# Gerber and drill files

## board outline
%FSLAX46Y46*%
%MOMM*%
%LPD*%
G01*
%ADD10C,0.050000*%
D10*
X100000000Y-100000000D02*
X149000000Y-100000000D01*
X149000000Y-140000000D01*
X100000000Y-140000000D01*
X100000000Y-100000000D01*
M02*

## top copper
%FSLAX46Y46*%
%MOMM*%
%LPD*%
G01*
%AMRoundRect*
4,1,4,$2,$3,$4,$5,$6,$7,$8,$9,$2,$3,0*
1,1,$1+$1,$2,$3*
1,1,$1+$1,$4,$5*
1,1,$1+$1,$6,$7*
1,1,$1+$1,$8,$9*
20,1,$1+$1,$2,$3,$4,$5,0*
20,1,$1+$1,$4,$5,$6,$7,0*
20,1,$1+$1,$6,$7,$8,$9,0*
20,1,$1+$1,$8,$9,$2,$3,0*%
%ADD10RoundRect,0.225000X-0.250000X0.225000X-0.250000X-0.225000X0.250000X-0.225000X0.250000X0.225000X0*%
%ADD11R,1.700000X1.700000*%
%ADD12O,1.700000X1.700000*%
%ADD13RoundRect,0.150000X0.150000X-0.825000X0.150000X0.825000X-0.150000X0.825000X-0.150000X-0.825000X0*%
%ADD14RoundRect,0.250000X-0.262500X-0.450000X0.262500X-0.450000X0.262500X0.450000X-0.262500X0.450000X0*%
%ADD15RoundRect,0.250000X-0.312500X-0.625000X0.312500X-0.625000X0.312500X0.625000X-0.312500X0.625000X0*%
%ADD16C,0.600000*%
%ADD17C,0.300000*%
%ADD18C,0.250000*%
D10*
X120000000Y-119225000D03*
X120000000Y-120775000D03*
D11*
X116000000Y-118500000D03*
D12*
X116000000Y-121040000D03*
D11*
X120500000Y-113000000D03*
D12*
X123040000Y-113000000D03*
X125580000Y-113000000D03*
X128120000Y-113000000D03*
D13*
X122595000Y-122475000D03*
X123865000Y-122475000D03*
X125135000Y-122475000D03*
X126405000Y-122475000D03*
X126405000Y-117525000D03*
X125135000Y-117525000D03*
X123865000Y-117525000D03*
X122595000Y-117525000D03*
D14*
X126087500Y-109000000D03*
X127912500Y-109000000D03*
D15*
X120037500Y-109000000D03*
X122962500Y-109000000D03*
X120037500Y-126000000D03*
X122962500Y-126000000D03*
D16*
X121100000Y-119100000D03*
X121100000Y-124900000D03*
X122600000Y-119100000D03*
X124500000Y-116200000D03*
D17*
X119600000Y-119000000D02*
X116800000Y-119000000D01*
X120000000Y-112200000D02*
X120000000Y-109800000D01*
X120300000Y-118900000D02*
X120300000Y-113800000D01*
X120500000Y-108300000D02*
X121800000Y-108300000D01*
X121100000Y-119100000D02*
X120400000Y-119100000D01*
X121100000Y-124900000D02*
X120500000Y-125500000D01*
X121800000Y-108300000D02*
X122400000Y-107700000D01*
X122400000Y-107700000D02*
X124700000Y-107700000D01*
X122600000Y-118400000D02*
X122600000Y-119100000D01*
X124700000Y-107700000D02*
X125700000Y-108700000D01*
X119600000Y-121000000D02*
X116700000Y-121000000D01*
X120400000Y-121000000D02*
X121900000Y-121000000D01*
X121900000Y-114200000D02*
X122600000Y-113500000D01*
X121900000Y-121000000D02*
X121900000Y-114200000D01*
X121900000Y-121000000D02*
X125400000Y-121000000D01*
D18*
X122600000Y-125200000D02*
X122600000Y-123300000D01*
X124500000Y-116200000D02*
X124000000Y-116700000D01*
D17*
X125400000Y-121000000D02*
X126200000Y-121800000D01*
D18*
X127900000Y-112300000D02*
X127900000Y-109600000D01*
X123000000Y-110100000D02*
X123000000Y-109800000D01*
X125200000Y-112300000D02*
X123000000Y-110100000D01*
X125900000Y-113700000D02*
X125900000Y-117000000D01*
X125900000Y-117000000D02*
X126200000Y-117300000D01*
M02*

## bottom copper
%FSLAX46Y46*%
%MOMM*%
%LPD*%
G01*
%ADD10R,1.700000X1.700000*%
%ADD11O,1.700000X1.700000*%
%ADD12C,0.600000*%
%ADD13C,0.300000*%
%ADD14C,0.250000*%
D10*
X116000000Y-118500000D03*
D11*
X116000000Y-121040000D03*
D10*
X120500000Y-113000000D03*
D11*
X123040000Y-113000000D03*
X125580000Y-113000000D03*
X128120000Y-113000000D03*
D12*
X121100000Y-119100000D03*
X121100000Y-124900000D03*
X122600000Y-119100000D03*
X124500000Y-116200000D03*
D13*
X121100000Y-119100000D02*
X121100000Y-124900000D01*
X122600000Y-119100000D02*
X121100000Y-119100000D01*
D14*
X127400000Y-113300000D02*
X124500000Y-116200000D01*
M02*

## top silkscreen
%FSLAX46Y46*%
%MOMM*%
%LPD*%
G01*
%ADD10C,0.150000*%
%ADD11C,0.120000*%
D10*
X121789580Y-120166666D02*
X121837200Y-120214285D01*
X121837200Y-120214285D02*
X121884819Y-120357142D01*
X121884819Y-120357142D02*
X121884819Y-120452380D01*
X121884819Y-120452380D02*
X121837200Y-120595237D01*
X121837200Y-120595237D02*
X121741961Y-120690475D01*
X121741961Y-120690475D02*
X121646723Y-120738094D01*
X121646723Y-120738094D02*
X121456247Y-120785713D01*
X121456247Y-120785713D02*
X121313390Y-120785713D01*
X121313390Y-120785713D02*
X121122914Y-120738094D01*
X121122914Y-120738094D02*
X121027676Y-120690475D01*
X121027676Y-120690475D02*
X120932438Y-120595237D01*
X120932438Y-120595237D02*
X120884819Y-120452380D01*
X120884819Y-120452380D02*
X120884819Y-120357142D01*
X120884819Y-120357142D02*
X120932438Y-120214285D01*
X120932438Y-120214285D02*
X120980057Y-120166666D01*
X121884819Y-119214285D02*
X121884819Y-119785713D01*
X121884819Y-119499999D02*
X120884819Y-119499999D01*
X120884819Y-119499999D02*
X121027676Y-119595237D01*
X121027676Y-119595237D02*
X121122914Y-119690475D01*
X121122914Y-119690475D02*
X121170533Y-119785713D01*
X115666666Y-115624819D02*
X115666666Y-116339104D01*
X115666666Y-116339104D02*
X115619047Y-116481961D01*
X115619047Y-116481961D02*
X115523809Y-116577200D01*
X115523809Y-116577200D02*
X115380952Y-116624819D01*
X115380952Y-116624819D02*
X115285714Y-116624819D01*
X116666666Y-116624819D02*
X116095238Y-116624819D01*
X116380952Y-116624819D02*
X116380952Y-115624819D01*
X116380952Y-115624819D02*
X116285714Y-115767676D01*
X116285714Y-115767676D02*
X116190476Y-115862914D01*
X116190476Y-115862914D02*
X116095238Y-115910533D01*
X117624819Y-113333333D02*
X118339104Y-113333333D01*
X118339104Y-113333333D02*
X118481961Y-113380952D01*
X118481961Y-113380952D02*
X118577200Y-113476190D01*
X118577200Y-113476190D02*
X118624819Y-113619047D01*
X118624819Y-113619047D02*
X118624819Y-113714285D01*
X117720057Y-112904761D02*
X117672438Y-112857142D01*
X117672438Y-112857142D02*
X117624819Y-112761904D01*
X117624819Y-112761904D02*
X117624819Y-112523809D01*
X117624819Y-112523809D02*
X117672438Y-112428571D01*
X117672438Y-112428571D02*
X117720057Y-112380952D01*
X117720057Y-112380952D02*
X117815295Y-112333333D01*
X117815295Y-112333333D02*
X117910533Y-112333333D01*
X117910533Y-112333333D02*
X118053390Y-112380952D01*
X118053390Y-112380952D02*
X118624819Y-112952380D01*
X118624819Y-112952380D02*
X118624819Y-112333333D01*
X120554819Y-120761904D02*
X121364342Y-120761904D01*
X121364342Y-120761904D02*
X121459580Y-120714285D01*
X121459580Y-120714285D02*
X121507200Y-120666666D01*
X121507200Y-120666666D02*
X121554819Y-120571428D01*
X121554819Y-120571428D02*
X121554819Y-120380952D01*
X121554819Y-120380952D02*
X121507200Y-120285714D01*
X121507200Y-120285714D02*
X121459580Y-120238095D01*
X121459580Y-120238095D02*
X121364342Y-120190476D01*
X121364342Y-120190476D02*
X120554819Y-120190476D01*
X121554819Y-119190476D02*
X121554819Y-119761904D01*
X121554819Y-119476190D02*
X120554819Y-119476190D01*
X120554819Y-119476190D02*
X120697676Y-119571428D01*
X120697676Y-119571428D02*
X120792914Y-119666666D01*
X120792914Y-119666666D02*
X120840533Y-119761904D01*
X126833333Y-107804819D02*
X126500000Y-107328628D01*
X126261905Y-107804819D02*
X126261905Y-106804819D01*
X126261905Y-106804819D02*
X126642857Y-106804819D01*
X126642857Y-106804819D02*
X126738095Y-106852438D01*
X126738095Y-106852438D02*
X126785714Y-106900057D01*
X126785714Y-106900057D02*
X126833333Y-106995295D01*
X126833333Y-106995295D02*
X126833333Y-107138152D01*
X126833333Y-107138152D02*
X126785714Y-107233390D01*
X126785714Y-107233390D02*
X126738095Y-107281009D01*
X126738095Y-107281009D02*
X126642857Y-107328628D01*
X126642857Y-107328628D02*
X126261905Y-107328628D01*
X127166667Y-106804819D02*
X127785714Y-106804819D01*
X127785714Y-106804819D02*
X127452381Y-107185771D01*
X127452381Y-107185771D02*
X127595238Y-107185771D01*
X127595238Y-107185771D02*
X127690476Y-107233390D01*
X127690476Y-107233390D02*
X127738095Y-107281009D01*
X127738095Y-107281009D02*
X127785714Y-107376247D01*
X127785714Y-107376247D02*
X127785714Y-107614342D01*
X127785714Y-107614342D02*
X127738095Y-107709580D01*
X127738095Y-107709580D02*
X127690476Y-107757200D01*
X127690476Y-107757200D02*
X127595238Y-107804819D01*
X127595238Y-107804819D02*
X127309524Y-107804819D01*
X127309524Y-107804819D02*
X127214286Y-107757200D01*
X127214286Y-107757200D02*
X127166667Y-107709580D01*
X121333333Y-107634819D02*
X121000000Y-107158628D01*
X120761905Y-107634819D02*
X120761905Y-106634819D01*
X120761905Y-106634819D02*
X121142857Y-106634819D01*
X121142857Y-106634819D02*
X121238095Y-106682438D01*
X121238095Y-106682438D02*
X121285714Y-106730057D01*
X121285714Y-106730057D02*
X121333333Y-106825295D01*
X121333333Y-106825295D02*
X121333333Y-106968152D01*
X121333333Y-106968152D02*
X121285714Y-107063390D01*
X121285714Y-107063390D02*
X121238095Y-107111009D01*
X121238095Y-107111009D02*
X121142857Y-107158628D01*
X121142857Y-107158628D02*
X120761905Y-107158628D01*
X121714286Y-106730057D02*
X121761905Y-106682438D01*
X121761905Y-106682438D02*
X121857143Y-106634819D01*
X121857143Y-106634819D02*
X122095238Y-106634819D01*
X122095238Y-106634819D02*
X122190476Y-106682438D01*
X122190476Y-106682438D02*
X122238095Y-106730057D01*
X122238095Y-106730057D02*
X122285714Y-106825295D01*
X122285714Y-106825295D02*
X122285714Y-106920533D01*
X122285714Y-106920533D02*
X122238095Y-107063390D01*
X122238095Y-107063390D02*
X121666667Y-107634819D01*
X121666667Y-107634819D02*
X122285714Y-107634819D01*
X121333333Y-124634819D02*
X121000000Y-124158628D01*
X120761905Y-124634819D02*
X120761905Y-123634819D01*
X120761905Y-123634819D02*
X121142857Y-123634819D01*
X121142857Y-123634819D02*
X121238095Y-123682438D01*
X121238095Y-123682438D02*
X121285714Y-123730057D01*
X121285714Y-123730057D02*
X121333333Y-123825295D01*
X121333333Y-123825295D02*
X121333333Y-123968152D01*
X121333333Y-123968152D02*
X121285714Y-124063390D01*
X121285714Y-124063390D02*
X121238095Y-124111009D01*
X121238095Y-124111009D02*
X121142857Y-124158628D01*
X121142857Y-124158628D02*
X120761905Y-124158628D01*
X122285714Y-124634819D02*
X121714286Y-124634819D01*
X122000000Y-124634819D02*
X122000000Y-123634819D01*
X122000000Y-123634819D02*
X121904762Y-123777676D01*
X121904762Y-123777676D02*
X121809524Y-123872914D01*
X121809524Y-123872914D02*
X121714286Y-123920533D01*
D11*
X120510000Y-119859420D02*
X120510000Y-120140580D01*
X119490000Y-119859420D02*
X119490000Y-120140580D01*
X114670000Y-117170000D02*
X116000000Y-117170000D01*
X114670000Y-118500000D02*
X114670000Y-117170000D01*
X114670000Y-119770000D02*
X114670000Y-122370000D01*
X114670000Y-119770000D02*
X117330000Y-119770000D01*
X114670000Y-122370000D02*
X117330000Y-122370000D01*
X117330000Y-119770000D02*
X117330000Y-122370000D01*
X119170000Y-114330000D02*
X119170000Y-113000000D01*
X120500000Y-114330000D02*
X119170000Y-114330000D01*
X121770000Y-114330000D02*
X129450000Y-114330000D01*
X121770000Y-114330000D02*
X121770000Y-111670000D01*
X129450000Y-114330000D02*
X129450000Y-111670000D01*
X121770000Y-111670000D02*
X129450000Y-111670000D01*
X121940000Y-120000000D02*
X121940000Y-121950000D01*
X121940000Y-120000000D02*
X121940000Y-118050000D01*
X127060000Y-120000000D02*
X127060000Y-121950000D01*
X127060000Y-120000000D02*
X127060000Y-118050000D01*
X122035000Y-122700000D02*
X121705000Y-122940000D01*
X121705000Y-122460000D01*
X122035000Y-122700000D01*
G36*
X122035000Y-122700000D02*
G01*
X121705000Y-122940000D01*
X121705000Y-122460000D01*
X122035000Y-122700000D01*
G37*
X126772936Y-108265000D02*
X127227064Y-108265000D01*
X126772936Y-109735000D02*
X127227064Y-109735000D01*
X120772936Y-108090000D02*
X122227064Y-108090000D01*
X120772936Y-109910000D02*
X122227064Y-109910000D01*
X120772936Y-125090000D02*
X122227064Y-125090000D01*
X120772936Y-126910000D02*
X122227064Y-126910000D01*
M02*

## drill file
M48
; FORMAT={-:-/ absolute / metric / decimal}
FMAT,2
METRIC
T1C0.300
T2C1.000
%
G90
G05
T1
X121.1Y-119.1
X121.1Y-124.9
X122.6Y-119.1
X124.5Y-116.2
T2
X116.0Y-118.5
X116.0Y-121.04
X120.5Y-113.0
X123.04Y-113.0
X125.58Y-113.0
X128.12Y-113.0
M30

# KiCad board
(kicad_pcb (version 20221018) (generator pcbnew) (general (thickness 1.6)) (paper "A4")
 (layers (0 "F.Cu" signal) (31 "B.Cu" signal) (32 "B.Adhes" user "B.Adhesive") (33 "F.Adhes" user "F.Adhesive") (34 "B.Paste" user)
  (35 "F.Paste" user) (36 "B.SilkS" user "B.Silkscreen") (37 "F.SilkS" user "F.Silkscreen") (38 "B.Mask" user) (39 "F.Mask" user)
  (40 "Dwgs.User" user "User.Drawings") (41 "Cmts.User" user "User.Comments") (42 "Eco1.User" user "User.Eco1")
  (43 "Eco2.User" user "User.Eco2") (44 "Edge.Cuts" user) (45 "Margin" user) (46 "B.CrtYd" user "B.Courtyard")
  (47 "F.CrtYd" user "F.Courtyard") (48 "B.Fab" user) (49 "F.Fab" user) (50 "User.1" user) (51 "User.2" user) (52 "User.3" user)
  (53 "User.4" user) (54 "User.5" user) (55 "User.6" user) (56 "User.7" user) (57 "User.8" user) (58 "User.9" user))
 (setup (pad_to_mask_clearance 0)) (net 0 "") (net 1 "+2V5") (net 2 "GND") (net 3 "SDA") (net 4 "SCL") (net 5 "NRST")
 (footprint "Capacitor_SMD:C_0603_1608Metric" (layer "F.Cu") (at 120 120 -90)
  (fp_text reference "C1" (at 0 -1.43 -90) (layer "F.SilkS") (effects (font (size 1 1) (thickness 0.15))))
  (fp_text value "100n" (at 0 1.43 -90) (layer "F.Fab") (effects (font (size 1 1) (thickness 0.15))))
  (fp_line (start -0.14058 -0.51) (end 0.14058 -0.51) (stroke (width 0.12) (type solid)) (layer "F.SilkS"))
  (fp_line (start -0.14058 0.51) (end 0.14058 0.51) (stroke (width 0.12) (type solid)) (layer "F.SilkS"))
  (pad "1" smd roundrect (at -0.775 0 270) (size 0.9 0.95) (layers "F.Cu" "F.Paste" "F.Mask") (roundrect_rratio 0.25) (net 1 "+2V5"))
  (pad "2" smd roundrect (at 0.775 0 270) (size 0.9 0.95) (layers "F.Cu" "F.Paste" "F.Mask") (roundrect_rratio 0.25) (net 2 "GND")))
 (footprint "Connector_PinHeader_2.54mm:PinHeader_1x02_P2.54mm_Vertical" (layer "F.Cu") (at 116 118.5)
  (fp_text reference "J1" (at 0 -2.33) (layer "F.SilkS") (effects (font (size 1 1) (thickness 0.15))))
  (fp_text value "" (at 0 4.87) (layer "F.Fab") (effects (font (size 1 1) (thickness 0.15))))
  (fp_line (start -1.33 -1.33) (end 0 -1.33) (stroke (width 0.12) (type solid)) (layer "F.SilkS"))
  (fp_line (start -1.33 0) (end -1.33 -1.33) (stroke (width 0.12) (type solid)) (layer "F.SilkS"))
  (fp_line (start -1.33 1.27) (end -1.33 3.87) (stroke (width 0.12) (type solid)) (layer "F.SilkS"))
  (fp_line (start -1.33 1.27) (end 1.33 1.27) (stroke (width 0.12) (type solid)) (layer "F.SilkS"))
  (fp_line (start -1.33 3.87) (end 1.33 3.87) (stroke (width 0.12) (type solid)) (layer "F.SilkS"))
  (fp_line (start 1.33 1.27) (end 1.33 3.87) (stroke (width 0.12) (type solid)) (layer "F.SilkS"))
  (pad "1" thru_hole rect (at 0 0) (size 1.7 1.7) (drill 1) (layers "*.Cu" "*.Mask") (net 1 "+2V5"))
  (pad "2" thru_hole oval (at 0 2.54) (size 1.7 1.7) (drill 1) (layers "*.Cu" "*.Mask") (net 2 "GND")))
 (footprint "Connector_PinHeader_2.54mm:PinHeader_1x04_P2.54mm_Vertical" (layer "F.Cu") (at 120.5 113 90)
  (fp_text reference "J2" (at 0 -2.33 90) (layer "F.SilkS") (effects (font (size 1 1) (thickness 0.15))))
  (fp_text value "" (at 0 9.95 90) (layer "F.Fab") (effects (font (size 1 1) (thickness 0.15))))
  (fp_line (start -1.33 -1.33) (end 0 -1.33) (stroke (width 0.12) (type solid)) (layer "F.SilkS"))
  (fp_line (start -1.33 0) (end -1.33 -1.33) (stroke (width 0.12) (type solid)) (layer "F.SilkS"))
  (fp_line (start -1.33 1.27) (end -1.33 8.95) (stroke (width 0.12) (type solid)) (layer "F.SilkS"))
  (fp_line (start -1.33 1.27) (end 1.33 1.27) (stroke (width 0.12) (type solid)) (layer "F.SilkS"))
  (fp_line (start -1.33 8.95) (end 1.33 8.95) (stroke (width 0.12) (type solid)) (layer "F.SilkS"))
  (fp_line (start 1.33 1.27) (end 1.33 8.95) (stroke (width 0.12) (type solid)) (layer "F.SilkS"))
  (pad "1" thru_hole rect (at 0 0 90) (size 1.7 1.7) (drill 1) (layers "*.Cu" "*.Mask") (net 1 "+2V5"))
  (pad "2" thru_hole oval (at 0 2.54 90) (size 1.7 1.7) (drill 1) (layers "*.Cu" "*.Mask") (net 2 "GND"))
  (pad "3" thru_hole oval (at 0 5.08 90) (size 1.7 1.7) (drill 1) (layers "*.Cu" "*.Mask") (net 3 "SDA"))
  (pad "4" thru_hole oval (at 0 7.62 90) (size 1.7 1.7) (drill 1) (layers "*.Cu" "*.Mask") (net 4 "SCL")))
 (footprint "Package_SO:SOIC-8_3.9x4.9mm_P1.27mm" (layer "F.Cu") (at 124.5 120 90)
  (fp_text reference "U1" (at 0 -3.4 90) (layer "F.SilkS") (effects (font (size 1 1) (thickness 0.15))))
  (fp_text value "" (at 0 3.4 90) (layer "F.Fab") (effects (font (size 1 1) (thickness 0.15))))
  (fp_line (start 0 -2.56) (end -1.95 -2.56) (stroke (width 0.12) (type solid)) (layer "F.SilkS"))
  (fp_line (start 0 -2.56) (end 1.95 -2.56) (stroke (width 0.12) (type solid)) (layer "F.SilkS"))
  (fp_line (start 0 2.56) (end -1.95 2.56) (stroke (width 0.12) (type solid)) (layer "F.SilkS"))
  (fp_line (start 0 2.56) (end 1.95 2.56) (stroke (width 0.12) (type solid)) (layer "F.SilkS"))
  (fp_poly
   (pts (xy -2.7 -2.465) (xy -2.94 -2.795) (xy -2.46 -2.795) (xy -2.7 -2.465)) (stroke (width 0.12) (type solid)) (fill solid)
   (layer "F.SilkS"))
  (pad "1" smd roundrect (at -2.475 -1.905 90) (size 1.95 0.6) (layers "F.Cu" "F.Paste" "F.Mask") (roundrect_rratio 0.25) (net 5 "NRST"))
  (pad "2" smd roundrect (at -2.475 -0.635 90) (size 1.95 0.6) (layers "F.Cu" "F.Paste" "F.Mask") (roundrect_rratio 0.25))
  (pad "3" smd roundrect (at -2.475 0.635 90) (size 1.95 0.6) (layers "F.Cu" "F.Paste" "F.Mask") (roundrect_rratio 0.25))
  (pad "4" smd roundrect (at -2.475 1.905 90) (size 1.95 0.6) (layers "F.Cu" "F.Paste" "F.Mask") (roundrect_rratio 0.25) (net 2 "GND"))
  (pad "5" smd roundrect (at 2.475 1.905 90) (size 1.95 0.6) (layers "F.Cu" "F.Paste" "F.Mask") (roundrect_rratio 0.25) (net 3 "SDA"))
  (pad "6" smd roundrect (at 2.475 0.635 90) (size 1.95 0.6) (layers "F.Cu" "F.Paste" "F.Mask") (roundrect_rratio 0.25))
  (pad "7" smd roundrect (at 2.475 -0.635 90) (size 1.95 0.6) (layers "F.Cu" "F.Paste" "F.Mask") (roundrect_rratio 0.25) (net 4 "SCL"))
  (pad "8" smd roundrect (at 2.475 -1.905 90) (size 1.95 0.6) (layers "F.Cu" "F.Paste" "F.Mask") (roundrect_rratio 0.25) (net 1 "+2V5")))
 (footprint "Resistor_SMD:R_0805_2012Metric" (layer "F.Cu") (at 127 109)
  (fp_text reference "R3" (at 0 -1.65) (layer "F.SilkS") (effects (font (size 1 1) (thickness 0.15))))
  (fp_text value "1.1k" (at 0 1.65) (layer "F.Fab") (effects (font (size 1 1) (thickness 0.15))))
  (fp_line (start -0.227064 -0.735) (end 0.227064 -0.735) (stroke (width 0.12) (type solid)) (layer "F.SilkS"))
  (fp_line (start -0.227064 0.735) (end 0.227064 0.735) (stroke (width 0.12) (type solid)) (layer "F.SilkS"))
  (pad "1" smd roundrect (at -0.9125 0) (size 1.025 1.4) (layers "F.Cu" "F.Paste" "F.Mask") (roundrect_rratio 0.243902) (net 1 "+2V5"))
  (pad "2" smd roundrect (at 0.9125 0) (size 1.025 1.4) (layers "F.Cu" "F.Paste" "F.Mask") (roundrect_rratio 0.243902) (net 4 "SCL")))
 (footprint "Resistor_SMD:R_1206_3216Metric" (layer "F.Cu") (at 121.5 109)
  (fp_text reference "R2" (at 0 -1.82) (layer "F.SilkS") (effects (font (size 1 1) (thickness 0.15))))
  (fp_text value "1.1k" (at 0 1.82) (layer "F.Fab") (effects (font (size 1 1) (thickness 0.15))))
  (fp_line (start -0.727064 -0.91) (end 0.727064 -0.91) (stroke (width 0.12) (type solid)) (layer "F.SilkS"))
  (fp_line (start -0.727064 0.91) (end 0.727064 0.91) (stroke (width 0.12) (type solid)) (layer "F.SilkS"))
  (pad "1" smd roundrect (at -1.4625 0) (size 1.125 1.75) (layers "F.Cu" "F.Paste" "F.Mask") (roundrect_rratio 0.222222) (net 1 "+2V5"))
  (pad "2" smd roundrect (at 1.4625 0) (size 1.125 1.75) (layers "F.Cu" "F.Paste" "F.Mask") (roundrect_rratio 0.222222) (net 3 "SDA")))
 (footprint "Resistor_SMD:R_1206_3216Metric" (layer "F.Cu") (at 121.5 126)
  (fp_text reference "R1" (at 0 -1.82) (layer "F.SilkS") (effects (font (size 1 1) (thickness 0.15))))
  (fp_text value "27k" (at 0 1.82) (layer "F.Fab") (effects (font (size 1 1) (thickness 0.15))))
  (fp_line (start -0.727064 -0.91) (end 0.727064 -0.91) (stroke (width 0.12) (type solid)) (layer "F.SilkS"))
  (fp_line (start -0.727064 0.91) (end 0.727064 0.91) (stroke (width 0.12) (type solid)) (layer "F.SilkS"))
  (pad "1" smd roundrect (at -1.4625 0) (size 1.125 1.75) (layers "F.Cu" "F.Paste" "F.Mask") (roundrect_rratio 0.222222) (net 1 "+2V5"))
  (pad "2" smd roundrect (at 1.4625 0) (size 1.125 1.75) (layers "F.Cu" "F.Paste" "F.Mask") (roundrect_rratio 0.222222) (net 5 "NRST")))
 (gr_rect (start 100 100) (end 149 140) (stroke (width 0.05) (type default)) (fill none) (layer "Edge.Cuts"))
 (segment (start 119.6 119) (end 116.8 119) (width 0.3) (layer "F.Cu") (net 1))
 (segment (start 120 112.2) (end 120 109.8) (width 0.3) (layer "F.Cu") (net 1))
 (segment (start 120.3 118.9) (end 120.3 113.8) (width 0.3) (layer "F.Cu") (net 1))
 (segment (start 120.5 108.3) (end 121.8 108.3) (width 0.3) (layer "F.Cu") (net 1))
 (segment (start 121.1 119.1) (end 120.4 119.1) (width 0.3) (layer "F.Cu") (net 1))
 (segment (start 121.1 124.9) (end 120.5 125.5) (width 0.3) (layer "F.Cu") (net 1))
 (segment (start 121.8 108.3) (end 122.4 107.7) (width 0.3) (layer "F.Cu") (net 1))
 (segment (start 122.4 107.7) (end 124.7 107.7) (width 0.3) (layer "F.Cu") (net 1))
 (segment (start 122.6 118.4) (end 122.6 119.1) (width 0.3) (layer "F.Cu") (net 1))
 (segment (start 124.7 107.7) (end 125.7 108.7) (width 0.3) (layer "F.Cu") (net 1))
 (via (at 121.1 119.1) (size 0.6) (drill 0.3) (layers "F.Cu" "B.Cu") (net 1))
 (via (at 121.1 124.9) (size 0.6) (drill 0.3) (layers "F.Cu" "B.Cu") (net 1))
 (via (at 122.6 119.1) (size 0.6) (drill 0.3) (layers "F.Cu" "B.Cu") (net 1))
 (segment (start 119.6 121) (end 116.7 121) (width 0.3) (layer "F.Cu") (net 2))
 (segment (start 120.4 121) (end 121.9 121) (width 0.3) (layer "F.Cu") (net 2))
 (segment (start 121.1 119.1) (end 121.1 124.9) (width 0.3) (layer "B.Cu") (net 1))
 (segment (start 121.9 114.2) (end 122.6 113.5) (width 0.3) (layer "F.Cu") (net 2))
 (segment (start 121.9 121) (end 121.9 114.2) (width 0.3) (layer "F.Cu") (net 2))
 (segment (start 121.9 121) (end 125.4 121) (width 0.3) (layer "F.Cu") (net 2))
 (segment (start 122.6 119.1) (end 121.1 119.1) (width 0.3) (layer "B.Cu") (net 1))
 (segment (start 122.6 125.2) (end 122.6 123.3) (width 0.25) (layer "F.Cu") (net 5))
 (segment (start 124.5 116.2) (end 124 116.7) (width 0.25) (layer "F.Cu") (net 4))
 (segment (start 125.4 121) (end 126.2 121.8) (width 0.3) (layer "F.Cu") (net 2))
 (segment (start 127.9 112.3) (end 127.9 109.6) (width 0.25) (layer "F.Cu") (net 4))
 (via (at 124.5 116.2) (size 0.6) (drill 0.3) (layers "F.Cu" "B.Cu") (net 4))
 (segment (start 123 110.1) (end 123 109.8) (width 0.25) (layer "F.Cu") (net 3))
 (segment (start 125.2 112.3) (end 123 110.1) (width 0.25) (layer "F.Cu") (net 3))
 (segment (start 125.9 113.7) (end 125.9 117) (width 0.25) (layer "F.Cu") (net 3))
 (segment (start 125.9 117) (end 126.2 117.3) (width 0.25) (layer "F.Cu") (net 3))
 (segment (start 127.4 113.3) (end 124.5 116.2) (width 0.25) (layer "B.Cu") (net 4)))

